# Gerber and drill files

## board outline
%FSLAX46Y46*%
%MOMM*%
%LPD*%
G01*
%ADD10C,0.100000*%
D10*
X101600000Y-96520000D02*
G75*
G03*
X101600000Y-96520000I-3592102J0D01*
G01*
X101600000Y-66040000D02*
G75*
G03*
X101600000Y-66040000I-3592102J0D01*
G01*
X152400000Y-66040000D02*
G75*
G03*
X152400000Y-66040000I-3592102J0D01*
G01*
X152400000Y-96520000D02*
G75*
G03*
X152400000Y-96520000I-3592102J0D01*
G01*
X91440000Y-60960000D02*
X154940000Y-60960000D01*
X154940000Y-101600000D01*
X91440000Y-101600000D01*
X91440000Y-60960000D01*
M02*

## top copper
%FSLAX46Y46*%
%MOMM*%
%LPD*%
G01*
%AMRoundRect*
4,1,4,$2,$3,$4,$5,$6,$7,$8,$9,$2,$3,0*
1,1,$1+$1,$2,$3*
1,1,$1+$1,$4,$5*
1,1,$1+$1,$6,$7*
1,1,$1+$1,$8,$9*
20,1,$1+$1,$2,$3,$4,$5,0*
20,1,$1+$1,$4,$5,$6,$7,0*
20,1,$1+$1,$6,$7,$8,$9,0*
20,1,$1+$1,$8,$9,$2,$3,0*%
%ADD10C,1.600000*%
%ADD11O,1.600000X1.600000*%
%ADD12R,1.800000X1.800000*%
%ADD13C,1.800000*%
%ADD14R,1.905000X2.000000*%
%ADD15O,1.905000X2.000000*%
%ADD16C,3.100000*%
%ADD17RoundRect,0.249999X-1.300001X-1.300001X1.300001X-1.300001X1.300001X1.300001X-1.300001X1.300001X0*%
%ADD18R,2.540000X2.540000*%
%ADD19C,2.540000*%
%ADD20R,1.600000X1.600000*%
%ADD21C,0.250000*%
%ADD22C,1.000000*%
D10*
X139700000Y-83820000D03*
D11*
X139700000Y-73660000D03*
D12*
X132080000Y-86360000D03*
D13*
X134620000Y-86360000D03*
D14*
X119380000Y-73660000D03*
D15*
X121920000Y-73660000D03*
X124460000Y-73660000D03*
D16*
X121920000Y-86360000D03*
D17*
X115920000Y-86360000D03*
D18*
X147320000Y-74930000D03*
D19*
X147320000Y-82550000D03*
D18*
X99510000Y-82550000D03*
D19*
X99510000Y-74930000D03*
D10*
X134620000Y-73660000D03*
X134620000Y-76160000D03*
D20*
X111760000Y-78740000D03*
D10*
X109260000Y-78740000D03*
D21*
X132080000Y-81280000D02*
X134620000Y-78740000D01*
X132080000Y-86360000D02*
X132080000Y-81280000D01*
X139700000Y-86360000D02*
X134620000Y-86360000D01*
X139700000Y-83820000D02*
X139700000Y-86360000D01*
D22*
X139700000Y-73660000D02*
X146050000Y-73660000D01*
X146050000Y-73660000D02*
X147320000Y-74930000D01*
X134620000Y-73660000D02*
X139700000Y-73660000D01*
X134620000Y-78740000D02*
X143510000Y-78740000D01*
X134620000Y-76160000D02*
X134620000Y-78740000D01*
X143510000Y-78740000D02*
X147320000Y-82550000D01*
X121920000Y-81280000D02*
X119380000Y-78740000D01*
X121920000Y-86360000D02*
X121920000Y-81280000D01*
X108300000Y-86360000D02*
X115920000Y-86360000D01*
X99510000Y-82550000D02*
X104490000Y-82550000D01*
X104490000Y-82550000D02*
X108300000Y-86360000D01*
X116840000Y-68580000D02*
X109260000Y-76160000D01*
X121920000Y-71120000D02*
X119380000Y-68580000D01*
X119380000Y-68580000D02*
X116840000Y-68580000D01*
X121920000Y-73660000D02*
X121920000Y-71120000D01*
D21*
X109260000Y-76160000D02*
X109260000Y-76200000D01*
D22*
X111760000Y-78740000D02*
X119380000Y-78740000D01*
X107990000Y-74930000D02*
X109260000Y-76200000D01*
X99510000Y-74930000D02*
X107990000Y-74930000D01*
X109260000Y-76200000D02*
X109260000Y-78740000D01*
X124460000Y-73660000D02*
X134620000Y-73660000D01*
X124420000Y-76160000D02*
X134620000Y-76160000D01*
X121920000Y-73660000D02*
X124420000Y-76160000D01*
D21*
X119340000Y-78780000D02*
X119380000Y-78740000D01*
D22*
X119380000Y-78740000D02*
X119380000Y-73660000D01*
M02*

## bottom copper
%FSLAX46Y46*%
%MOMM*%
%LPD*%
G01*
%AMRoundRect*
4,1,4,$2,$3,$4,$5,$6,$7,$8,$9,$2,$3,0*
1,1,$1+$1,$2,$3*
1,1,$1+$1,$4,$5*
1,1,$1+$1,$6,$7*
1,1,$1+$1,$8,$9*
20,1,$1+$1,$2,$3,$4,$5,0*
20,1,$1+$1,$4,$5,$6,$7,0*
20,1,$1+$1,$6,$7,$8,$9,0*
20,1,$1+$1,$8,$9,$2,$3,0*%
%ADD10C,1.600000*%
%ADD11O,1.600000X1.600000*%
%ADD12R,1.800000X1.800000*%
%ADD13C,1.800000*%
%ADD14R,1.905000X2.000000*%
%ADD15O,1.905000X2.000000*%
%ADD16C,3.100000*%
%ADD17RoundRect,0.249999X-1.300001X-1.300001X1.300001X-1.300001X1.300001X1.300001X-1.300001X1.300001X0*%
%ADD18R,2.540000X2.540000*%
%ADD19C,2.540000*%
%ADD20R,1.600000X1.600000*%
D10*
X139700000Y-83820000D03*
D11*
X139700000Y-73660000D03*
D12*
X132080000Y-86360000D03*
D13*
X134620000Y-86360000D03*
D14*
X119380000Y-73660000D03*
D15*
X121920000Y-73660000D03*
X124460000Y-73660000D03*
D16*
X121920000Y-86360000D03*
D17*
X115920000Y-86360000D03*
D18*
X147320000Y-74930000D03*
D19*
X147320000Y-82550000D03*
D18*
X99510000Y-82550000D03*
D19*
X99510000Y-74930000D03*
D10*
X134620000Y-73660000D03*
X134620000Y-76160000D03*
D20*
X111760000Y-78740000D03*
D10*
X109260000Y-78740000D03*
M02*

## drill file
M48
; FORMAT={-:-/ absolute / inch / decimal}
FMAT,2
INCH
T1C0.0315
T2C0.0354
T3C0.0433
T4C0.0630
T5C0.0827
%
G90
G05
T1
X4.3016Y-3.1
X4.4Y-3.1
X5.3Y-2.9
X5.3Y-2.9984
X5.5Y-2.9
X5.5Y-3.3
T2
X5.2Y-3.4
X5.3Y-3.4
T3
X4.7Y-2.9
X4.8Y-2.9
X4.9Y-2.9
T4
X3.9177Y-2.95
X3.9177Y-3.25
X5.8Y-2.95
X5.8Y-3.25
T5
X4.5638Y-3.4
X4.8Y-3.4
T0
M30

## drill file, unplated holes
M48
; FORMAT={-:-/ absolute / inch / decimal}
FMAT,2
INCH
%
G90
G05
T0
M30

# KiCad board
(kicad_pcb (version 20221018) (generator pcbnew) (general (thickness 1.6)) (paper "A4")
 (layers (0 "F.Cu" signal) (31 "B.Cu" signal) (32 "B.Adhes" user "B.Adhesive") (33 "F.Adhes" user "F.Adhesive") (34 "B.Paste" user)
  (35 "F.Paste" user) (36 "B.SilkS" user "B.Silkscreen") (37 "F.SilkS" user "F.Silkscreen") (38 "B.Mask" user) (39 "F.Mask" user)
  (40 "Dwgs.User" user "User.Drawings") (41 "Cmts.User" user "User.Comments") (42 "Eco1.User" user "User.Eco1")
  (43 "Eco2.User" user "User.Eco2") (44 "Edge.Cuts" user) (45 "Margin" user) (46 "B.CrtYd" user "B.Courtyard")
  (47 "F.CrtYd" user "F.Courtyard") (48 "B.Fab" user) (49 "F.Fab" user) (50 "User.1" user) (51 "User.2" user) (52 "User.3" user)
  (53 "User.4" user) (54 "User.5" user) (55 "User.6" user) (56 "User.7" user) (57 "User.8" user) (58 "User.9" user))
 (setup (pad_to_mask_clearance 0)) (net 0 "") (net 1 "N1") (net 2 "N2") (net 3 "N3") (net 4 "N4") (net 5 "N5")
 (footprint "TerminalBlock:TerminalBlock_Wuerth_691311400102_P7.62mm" (layer "F.Cu") (at 147.32 74.93 -90)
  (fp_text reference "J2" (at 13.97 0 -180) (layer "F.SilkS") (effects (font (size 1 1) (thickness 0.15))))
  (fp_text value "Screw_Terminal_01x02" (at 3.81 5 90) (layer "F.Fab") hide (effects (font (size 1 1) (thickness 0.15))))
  (pad "1" thru_hole rect (at 0 0 270) (size 2.54 2.54) (drill 1.6) (layers "*.Cu" "*.Mask") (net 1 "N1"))
  (pad "2" thru_hole circle (at 7.62 0 270) (size 2.54 2.54) (drill 1.6) (layers "*.Cu" "*.Mask") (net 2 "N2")))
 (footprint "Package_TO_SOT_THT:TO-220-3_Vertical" (layer "F.Cu") (at 119.38 73.66)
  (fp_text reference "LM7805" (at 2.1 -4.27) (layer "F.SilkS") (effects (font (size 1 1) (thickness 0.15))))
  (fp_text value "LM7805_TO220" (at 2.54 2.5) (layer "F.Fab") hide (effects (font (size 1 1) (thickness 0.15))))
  (pad "1" thru_hole rect (at 0 0) (size 1.905 2) (drill 1.1) (layers "*.Cu" "*.Mask") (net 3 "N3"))
  (pad "2" thru_hole oval (at 2.54 0) (size 1.905 2) (drill 1.1) (layers "*.Cu" "*.Mask") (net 2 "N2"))
  (pad "3" thru_hole oval (at 5.08 0) (size 1.905 2) (drill 1.1) (layers "*.Cu" "*.Mask") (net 1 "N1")))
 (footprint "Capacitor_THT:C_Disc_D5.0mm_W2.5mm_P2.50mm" (layer "F.Cu") (at 134.62 73.66 -90)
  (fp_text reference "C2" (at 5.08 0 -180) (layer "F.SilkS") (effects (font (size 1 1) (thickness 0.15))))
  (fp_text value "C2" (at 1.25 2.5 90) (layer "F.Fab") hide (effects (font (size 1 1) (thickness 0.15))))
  (pad "1" thru_hole circle (at 0 0 270) (size 1.6 1.6) (drill 0.8) (layers "*.Cu" "*.Mask") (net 1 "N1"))
  (pad "2" thru_hole circle (at 2.5 0 270) (size 1.6 1.6) (drill 0.8) (layers "*.Cu" "*.Mask") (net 2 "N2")))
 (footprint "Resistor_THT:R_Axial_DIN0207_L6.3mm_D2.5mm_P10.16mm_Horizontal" (layer "F.Cu") (at 139.7 83.82 90)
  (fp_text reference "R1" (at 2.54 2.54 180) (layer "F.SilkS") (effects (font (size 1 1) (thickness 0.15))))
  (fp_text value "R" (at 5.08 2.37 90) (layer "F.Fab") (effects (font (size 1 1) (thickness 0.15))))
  (pad "1" thru_hole circle (at 0 0 90) (size 1.6 1.6) (drill 0.8) (layers "*.Cu" "*.Mask") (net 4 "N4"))
  (pad "2" thru_hole oval (at 10.16 0 90) (size 1.6 1.6) (drill 0.8) (layers "*.Cu" "*.Mask") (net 1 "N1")))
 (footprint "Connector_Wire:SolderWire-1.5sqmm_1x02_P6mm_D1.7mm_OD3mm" (layer "F.Cu") (at 115.92 86.36)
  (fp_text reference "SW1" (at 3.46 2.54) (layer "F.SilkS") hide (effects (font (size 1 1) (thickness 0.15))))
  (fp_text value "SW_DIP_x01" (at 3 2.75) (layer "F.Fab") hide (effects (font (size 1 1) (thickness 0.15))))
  (pad "1" thru_hole roundrect (at 0 0) (size 3.1 3.1) (drill 2.1) (layers "*.Cu" "*.Mask") (roundrect_rratio 0.08064483871) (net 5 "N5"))
  (pad "2" thru_hole circle (at 6 0) (size 3.1 3.1) (drill 2.1) (layers "*.Cu" "*.Mask") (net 3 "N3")))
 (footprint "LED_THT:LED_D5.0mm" (layer "F.Cu") (at 132.08 86.36)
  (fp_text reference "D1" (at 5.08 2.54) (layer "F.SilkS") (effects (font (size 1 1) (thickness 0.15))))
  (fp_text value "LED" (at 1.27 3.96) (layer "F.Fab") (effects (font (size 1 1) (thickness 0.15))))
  (pad "1" thru_hole rect (at 0 0) (size 1.8 1.8) (drill 0.9) (layers "*.Cu" "*.Mask") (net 2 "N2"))
  (pad "2" thru_hole circle (at 2.54 0) (size 1.8 1.8) (drill 0.9) (layers "*.Cu" "*.Mask") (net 4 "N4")))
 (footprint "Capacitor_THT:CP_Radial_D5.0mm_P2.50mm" (layer "F.Cu") (at 111.76 78.74 180)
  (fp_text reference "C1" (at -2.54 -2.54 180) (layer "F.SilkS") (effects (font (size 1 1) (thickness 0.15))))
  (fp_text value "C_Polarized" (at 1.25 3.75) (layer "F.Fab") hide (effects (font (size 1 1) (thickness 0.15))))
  (pad "1" thru_hole rect (at 0 0 180) (size 1.6 1.6) (drill 0.8) (layers "*.Cu" "*.Mask") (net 3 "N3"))
  (pad "2" thru_hole circle (at 2.5 0 180) (size 1.6 1.6) (drill 0.8) (layers "*.Cu" "*.Mask") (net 2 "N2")))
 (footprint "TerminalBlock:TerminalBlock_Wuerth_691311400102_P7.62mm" (layer "F.Cu") (at 99.51 82.55 90)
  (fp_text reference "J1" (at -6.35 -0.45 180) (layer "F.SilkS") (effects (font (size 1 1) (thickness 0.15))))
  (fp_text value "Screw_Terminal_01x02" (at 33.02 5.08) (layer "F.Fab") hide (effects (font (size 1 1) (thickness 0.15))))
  (pad "1" thru_hole rect (at 0 0 90) (size 2.54 2.54) (drill 1.6) (layers "*.Cu" "*.Mask") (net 5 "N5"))
  (pad "2" thru_hole circle (at 7.62 0 90) (size 2.54 2.54) (drill 1.6) (layers "*.Cu" "*.Mask") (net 2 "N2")))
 (gr_circle (center 98.007898 96.52) (end 100.547898 99.06) (stroke (width 0.1) (type default)) (fill none) (layer "Edge.Cuts"))
 (gr_circle (center 98.007898 66.04) (end 100.547898 68.58) (stroke (width 0.1) (type default)) (fill none) (layer "Edge.Cuts"))
 (gr_circle (center 148.807898 96.52) (end 151.347898 99.06) (stroke (width 0.1) (type default)) (fill none) (layer "Edge.Cuts"))
 (gr_circle (center 148.807898 66.04) (end 151.347898 68.58) (stroke (width 0.1) (type default)) (fill none) (layer "Edge.Cuts"))
 (gr_rect (start 91.44 60.96) (end 154.94 101.6) (stroke (width 0.1) (type default)) (fill none) (layer "Edge.Cuts"))
 (segment (start 121.92 81.28) (end 119.38 78.74) (width 1) (layer "F.Cu") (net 3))
 (segment (start 119.38 78.74) (end 119.38 73.66) (width 1) (layer "F.Cu") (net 3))
 (segment (start 119.34 78.78) (end 119.38 78.74) (width 0.25) (layer "F.Cu") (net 3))
 (segment (start 111.76 78.74) (end 119.38 78.74) (width 1) (layer "F.Cu") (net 3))
 (segment (start 121.92 86.36) (end 121.92 81.28) (width 1) (layer "F.Cu") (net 3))
 (segment (start 124.46 73.66) (end 134.62 73.66) (width 1) (layer "F.Cu") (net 1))
 (segment (start 146.05 73.66) (end 147.32 74.93) (width 1) (layer "F.Cu") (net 1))
 (segment (start 139.7 73.66) (end 146.05 73.66) (width 1) (layer "F.Cu") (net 1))
 (segment (start 134.62 73.66) (end 139.7 73.66) (width 1) (layer "F.Cu") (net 1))
 (segment (start 108.3 86.36) (end 115.92 86.36) (width 1) (layer "F.Cu") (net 5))
 (segment (start 99.51 82.55) (end 104.49 82.55) (width 1) (layer "F.Cu") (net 5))
 (segment (start 104.49 82.55) (end 108.3 86.36) (width 1) (layer "F.Cu") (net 5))
 (segment (start 134.62 76.16) (end 134.62 78.74) (width 1) (layer "F.Cu") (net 2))
 (segment (start 121.92 73.66) (end 124.42 76.16) (width 1) (layer "F.Cu") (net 2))
 (segment (start 121.92 71.12) (end 119.38 68.58) (width 1) (layer "F.Cu") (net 2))
 (segment (start 109.26 76.2) (end 109.26 78.74) (width 1) (layer "F.Cu") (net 2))
 (segment (start 109.26 76.16) (end 109.26 76.2) (width 0.25) (layer "F.Cu") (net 2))
 (segment (start 99.51 74.93) (end 107.99 74.93) (width 1) (layer "F.Cu") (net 2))
 (segment (start 121.92 73.66) (end 121.92 71.12) (width 1) (layer "F.Cu") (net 2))
 (segment (start 119.38 68.58) (end 116.84 68.58) (width 1) (layer "F.Cu") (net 2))
 (segment (start 132.08 81.28) (end 134.62 78.74) (width 0.25) (layer "F.Cu") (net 2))
 (segment (start 107.99 74.93) (end 109.26 76.2) (width 1) (layer "F.Cu") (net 2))
 (segment (start 116.84 68.58) (end 109.26 76.16) (width 1) (layer "F.Cu") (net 2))
 (segment (start 132.08 86.36) (end 132.08 81.28) (width 0.25) (layer "F.Cu") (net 2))
 (segment (start 143.51 78.74) (end 147.32 82.55) (width 1) (layer "F.Cu") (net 2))
 (segment (start 124.42 76.16) (end 134.62 76.16) (width 1) (layer "F.Cu") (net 2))
 (segment (start 134.62 78.74) (end 143.51 78.74) (width 1) (layer "F.Cu") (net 2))
 (segment (start 139.7 86.36) (end 134.62 86.36) (width 0.25) (layer "F.Cu") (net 4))
 (segment (start 139.7 83.82) (end 139.7 86.36) (width 0.25) (layer "F.Cu") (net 4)))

